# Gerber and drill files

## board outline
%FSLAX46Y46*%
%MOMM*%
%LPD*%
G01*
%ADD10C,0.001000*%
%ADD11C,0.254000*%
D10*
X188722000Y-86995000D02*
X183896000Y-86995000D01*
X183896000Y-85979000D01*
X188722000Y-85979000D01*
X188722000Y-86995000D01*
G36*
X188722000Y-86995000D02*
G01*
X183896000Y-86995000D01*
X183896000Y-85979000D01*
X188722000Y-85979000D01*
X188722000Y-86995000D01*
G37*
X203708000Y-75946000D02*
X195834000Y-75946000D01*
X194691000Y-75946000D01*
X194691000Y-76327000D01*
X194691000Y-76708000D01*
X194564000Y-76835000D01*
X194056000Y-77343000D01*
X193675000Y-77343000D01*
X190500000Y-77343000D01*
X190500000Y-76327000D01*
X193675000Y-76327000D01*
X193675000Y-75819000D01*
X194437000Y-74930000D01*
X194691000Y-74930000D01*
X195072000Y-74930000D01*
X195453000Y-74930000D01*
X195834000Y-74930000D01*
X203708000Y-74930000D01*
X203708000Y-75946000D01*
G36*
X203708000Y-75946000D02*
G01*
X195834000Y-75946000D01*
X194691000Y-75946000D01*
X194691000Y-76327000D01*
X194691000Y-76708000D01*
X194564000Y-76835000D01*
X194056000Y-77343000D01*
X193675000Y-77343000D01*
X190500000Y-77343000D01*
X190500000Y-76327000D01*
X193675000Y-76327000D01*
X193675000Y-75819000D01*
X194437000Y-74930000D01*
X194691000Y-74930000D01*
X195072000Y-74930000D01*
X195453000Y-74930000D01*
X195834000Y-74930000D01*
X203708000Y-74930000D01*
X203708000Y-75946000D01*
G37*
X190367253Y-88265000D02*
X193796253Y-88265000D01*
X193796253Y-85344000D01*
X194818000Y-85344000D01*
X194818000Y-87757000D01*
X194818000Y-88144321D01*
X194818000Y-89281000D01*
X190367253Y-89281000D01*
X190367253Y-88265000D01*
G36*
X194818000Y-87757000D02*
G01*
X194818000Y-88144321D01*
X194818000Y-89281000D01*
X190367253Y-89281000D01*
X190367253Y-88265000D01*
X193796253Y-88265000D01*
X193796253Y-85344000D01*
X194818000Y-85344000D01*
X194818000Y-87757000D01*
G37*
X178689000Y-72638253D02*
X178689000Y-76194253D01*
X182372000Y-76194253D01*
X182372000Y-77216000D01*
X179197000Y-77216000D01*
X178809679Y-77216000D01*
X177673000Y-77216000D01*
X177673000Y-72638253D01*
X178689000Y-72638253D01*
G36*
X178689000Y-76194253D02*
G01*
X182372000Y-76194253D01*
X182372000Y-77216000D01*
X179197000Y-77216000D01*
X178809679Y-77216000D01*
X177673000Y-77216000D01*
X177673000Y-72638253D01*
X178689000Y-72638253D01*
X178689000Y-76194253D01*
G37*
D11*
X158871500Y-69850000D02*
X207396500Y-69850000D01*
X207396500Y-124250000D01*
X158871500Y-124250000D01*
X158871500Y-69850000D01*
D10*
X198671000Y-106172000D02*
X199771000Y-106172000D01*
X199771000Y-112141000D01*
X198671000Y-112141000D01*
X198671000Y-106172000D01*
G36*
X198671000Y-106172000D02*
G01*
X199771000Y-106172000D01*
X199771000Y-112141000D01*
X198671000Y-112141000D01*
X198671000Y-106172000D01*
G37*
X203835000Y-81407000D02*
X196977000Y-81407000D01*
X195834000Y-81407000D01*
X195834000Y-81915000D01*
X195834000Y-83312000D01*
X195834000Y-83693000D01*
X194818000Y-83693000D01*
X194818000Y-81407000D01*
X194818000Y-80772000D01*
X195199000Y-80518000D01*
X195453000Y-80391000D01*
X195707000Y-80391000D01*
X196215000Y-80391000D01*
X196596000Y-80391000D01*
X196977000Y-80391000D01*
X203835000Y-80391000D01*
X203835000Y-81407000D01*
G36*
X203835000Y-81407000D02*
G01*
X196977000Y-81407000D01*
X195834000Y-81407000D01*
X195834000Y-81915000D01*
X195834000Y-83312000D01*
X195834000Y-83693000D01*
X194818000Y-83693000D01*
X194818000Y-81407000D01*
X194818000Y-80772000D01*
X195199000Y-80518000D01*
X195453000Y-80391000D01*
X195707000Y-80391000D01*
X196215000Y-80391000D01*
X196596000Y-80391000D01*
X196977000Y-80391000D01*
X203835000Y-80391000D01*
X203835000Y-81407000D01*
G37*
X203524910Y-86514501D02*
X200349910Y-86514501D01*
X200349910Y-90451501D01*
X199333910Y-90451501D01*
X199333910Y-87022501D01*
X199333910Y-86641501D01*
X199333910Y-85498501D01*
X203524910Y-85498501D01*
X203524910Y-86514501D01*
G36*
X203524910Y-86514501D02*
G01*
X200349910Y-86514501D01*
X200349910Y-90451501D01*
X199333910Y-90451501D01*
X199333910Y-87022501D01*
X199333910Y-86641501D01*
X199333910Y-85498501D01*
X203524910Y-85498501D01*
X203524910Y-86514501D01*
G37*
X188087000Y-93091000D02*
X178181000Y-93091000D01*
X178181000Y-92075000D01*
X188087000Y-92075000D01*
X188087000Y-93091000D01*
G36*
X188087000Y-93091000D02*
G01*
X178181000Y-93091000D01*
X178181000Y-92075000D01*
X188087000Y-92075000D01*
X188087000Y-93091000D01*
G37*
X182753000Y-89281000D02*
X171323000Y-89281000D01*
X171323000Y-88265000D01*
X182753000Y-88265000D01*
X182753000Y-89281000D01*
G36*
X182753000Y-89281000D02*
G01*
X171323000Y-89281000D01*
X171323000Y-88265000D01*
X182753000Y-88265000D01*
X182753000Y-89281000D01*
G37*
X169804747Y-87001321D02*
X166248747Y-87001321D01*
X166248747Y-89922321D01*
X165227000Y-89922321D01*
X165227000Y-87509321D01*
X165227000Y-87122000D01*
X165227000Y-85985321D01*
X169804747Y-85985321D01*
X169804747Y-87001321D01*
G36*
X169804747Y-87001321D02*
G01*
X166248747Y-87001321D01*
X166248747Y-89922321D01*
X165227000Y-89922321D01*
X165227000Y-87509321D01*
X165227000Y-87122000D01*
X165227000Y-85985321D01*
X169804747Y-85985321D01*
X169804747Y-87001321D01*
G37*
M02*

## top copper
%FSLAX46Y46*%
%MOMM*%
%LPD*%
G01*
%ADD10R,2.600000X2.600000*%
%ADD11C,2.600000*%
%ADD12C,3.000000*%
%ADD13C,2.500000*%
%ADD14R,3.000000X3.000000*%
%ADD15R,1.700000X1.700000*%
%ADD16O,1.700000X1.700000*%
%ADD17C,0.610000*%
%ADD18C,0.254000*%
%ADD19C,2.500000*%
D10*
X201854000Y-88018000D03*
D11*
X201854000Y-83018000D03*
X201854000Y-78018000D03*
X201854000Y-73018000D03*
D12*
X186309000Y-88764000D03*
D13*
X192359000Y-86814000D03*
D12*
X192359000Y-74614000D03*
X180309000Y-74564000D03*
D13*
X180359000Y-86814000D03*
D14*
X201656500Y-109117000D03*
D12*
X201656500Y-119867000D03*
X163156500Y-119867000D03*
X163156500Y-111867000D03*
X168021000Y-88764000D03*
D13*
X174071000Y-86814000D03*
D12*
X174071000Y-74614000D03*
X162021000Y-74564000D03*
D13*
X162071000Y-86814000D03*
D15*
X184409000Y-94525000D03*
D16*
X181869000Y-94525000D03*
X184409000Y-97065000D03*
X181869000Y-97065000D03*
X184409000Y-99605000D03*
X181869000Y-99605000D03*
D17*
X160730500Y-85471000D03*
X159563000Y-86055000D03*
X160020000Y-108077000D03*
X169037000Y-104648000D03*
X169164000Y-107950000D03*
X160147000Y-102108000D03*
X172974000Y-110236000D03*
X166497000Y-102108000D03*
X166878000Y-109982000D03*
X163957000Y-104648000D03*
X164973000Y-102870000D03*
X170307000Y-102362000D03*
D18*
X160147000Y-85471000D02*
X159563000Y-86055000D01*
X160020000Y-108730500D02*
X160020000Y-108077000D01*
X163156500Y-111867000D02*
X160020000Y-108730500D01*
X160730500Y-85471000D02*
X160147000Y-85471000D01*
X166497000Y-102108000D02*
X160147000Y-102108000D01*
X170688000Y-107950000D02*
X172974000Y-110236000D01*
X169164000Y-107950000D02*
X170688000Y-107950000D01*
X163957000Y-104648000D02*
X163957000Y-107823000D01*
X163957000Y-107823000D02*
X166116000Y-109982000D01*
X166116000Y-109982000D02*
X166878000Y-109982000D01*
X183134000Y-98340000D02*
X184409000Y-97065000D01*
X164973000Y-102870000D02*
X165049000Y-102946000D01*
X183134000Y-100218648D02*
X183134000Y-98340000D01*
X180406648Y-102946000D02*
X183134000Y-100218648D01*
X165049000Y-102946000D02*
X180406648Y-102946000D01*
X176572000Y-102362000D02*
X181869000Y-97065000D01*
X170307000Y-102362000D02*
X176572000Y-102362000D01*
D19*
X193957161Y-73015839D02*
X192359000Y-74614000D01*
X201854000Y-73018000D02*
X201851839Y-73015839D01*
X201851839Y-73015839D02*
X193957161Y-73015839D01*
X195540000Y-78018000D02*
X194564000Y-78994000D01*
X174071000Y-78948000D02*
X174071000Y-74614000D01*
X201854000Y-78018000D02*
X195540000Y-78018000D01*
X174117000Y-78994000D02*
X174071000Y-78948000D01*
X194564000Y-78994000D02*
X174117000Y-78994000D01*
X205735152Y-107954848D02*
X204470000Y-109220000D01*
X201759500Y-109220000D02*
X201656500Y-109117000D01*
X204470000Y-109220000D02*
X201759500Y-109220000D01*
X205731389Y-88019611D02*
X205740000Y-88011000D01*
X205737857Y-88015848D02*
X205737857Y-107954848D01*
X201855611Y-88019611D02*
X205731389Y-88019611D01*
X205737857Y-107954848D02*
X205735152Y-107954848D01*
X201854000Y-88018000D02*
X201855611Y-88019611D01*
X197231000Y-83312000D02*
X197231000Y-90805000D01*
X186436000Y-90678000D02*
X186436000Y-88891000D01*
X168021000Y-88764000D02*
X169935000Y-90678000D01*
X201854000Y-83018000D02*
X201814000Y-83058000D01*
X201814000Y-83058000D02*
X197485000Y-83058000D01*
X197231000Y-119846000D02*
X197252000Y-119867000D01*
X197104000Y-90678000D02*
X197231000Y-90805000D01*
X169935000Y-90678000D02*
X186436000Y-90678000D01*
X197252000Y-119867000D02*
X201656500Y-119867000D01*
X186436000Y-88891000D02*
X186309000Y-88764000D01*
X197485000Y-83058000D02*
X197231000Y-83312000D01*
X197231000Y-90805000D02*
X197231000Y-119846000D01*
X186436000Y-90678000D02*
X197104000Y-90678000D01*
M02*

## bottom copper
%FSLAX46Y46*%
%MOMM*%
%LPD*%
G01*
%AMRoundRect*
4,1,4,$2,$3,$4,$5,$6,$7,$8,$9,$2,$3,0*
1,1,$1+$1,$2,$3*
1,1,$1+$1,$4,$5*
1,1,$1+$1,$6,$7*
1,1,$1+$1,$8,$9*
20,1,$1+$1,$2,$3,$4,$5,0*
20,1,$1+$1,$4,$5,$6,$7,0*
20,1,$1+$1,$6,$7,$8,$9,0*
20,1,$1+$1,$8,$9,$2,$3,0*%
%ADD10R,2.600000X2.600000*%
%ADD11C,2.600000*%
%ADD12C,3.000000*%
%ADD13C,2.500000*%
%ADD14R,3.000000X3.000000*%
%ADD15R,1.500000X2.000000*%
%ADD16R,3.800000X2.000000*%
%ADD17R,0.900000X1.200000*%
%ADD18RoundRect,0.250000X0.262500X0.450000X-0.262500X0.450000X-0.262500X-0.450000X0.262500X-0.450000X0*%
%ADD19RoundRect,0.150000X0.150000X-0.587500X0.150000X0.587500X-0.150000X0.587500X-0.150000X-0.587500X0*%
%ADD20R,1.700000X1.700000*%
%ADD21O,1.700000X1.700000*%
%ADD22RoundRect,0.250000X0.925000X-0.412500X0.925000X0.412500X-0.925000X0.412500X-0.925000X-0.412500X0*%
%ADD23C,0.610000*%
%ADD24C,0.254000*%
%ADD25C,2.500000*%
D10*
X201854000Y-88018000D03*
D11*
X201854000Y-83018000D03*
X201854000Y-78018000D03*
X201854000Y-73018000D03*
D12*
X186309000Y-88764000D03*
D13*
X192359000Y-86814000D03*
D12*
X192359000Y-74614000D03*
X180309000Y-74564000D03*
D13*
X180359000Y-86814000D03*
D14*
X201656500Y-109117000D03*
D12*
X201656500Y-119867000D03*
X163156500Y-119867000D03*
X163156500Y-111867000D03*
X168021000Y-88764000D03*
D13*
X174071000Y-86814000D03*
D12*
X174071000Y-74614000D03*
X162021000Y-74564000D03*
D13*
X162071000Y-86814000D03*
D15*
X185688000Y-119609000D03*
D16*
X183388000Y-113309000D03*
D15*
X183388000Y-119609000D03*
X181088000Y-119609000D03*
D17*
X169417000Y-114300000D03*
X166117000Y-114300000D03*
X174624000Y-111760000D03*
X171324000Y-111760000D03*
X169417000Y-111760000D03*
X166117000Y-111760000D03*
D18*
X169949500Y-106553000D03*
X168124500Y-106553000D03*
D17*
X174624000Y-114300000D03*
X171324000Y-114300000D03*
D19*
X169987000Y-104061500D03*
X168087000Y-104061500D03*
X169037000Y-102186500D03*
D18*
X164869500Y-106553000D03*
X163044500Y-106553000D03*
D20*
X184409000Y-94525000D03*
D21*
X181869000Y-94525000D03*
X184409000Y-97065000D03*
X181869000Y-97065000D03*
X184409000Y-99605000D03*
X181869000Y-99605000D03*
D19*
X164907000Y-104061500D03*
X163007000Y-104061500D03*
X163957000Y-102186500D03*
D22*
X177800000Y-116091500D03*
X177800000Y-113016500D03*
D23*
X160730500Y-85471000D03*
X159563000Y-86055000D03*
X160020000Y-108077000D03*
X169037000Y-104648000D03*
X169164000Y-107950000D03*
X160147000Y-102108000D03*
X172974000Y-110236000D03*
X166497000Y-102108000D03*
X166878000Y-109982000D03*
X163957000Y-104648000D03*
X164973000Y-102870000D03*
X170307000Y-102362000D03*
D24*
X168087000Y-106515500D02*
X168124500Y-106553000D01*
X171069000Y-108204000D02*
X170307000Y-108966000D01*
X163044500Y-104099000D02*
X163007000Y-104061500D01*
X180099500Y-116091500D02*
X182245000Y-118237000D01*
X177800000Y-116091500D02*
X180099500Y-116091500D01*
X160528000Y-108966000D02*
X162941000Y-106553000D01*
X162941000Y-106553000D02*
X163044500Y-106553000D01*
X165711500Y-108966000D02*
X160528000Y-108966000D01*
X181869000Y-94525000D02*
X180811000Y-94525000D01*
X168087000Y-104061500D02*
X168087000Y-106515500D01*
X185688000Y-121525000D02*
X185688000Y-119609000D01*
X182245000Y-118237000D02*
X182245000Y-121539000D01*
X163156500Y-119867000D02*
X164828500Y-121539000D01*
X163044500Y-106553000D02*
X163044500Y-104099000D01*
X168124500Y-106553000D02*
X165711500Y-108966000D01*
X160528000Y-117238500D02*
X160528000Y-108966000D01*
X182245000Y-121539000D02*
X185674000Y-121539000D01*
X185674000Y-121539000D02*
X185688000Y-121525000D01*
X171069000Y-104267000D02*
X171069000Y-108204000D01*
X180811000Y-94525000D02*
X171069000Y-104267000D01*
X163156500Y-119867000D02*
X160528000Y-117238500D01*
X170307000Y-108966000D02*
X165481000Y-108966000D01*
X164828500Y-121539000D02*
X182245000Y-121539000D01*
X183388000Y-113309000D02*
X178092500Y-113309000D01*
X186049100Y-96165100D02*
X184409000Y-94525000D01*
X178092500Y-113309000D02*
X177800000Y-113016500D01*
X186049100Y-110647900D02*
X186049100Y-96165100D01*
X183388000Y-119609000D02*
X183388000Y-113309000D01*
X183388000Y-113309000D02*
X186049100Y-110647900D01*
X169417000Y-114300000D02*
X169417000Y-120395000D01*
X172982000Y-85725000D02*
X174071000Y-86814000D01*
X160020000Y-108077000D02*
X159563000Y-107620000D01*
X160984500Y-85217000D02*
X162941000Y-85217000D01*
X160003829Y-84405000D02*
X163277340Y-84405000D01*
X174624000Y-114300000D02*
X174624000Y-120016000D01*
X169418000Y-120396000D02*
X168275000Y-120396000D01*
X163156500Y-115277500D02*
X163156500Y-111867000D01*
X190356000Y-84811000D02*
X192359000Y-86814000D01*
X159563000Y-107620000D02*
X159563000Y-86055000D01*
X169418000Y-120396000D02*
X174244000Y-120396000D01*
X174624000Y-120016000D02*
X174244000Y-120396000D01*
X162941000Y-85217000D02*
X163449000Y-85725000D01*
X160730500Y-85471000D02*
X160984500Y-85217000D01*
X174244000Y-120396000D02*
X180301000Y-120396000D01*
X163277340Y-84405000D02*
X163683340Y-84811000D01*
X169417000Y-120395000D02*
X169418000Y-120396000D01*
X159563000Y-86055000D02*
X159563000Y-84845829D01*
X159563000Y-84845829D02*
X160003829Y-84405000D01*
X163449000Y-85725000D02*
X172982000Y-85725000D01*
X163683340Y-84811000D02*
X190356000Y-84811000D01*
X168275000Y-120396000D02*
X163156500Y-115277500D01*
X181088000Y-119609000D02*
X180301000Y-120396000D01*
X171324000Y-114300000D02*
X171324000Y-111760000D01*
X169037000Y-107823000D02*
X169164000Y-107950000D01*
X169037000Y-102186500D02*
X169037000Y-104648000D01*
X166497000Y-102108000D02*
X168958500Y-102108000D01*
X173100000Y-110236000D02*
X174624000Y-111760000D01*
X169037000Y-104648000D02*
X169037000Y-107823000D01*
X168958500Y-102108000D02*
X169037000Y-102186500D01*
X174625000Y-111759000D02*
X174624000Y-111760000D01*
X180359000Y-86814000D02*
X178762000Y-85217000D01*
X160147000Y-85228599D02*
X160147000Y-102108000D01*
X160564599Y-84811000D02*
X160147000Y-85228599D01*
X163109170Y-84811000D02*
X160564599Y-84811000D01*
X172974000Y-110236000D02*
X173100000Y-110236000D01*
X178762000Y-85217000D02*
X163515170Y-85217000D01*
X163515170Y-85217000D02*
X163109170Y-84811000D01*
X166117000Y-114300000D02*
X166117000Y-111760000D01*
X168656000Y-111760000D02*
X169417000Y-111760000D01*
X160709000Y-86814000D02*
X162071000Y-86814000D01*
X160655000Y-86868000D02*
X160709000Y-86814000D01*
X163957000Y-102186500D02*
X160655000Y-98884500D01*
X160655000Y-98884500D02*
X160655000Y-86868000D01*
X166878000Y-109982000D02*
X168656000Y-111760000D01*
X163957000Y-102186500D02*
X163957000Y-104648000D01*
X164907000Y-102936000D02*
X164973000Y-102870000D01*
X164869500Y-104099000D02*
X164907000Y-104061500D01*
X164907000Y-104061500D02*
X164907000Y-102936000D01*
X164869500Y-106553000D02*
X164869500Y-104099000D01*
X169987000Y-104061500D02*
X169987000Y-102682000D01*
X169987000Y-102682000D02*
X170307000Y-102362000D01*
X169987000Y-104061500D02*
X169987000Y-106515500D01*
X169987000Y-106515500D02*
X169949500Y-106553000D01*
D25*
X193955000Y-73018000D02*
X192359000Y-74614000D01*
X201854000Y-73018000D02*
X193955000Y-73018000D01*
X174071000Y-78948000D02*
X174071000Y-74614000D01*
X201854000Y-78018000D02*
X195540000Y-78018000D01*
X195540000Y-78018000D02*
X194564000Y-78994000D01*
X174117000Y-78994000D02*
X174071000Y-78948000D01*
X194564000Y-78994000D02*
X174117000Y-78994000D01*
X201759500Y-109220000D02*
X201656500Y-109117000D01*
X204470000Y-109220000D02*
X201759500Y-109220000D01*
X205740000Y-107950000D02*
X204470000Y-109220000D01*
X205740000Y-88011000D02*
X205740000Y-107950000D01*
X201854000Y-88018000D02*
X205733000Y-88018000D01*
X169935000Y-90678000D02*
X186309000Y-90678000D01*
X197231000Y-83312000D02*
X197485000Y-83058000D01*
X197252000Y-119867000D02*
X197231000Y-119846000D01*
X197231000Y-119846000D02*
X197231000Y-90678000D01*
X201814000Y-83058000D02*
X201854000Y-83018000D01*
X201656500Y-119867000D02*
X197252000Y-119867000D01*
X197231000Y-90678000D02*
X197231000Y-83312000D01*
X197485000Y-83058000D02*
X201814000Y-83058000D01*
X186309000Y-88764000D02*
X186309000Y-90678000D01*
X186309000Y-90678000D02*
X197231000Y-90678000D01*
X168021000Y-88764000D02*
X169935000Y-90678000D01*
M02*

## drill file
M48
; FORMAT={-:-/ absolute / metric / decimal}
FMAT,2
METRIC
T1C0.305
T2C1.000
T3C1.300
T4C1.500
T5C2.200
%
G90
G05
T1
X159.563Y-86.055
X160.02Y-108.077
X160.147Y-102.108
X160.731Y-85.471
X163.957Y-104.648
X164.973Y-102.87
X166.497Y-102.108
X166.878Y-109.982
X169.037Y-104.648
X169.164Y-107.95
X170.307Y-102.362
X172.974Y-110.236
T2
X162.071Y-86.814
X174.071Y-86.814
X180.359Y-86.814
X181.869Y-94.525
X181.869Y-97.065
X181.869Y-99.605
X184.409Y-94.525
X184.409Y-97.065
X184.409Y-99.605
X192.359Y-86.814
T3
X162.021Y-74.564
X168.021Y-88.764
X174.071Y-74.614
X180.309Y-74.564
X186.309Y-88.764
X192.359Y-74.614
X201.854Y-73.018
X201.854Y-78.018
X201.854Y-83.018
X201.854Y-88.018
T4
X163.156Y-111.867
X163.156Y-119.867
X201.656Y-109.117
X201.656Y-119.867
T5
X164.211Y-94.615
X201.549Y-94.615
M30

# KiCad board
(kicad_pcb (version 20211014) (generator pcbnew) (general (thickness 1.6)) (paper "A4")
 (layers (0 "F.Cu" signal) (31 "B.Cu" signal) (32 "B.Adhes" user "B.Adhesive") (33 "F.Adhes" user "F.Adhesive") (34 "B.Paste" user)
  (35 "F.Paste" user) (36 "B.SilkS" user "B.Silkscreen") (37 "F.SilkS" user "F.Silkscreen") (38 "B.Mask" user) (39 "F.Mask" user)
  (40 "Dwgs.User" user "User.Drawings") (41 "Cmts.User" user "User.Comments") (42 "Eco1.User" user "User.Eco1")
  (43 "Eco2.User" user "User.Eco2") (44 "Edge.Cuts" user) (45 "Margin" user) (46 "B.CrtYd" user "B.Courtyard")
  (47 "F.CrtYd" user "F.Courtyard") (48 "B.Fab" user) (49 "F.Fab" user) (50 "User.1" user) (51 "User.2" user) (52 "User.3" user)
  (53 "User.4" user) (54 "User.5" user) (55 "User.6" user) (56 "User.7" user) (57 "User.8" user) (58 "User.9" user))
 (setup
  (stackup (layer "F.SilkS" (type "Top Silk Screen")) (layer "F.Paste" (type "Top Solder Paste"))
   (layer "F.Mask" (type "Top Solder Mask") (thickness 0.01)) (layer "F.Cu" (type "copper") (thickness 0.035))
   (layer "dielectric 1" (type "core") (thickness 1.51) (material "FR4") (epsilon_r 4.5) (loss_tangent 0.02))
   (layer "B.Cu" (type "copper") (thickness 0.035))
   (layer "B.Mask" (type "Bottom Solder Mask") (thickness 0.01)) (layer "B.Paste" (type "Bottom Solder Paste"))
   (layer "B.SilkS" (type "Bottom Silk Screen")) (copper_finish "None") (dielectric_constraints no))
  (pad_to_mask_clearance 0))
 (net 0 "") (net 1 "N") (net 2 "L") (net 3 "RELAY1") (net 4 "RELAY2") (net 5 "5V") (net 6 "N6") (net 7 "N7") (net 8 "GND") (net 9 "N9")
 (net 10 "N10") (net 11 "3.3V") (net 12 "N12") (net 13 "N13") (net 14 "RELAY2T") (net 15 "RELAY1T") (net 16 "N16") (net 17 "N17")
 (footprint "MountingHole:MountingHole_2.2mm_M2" (layer "F.Cu") (at 164.211 94.615)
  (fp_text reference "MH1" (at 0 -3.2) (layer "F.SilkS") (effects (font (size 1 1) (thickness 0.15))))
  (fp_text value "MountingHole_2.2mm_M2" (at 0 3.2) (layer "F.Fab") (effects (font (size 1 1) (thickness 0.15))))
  (pad "" np_thru_hole circle (at 0 0) (size 2.2 2.2) (drill 2.2) (layers *.Cu *.Mask)))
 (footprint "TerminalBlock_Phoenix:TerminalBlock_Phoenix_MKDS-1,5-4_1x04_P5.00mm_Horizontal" (layer "F.Cu") (at 201.854 88.018 90)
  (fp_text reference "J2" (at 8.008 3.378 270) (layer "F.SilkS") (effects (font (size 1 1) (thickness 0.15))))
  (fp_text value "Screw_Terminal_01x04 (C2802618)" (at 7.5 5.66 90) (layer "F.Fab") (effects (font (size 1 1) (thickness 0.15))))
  (pad "1" thru_hole rect (at 0 0 90) (size 2.6 2.6) (drill 1.3) (layers *.Cu *.Mask) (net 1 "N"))
  (pad "2" thru_hole circle (at 5 0 90) (size 2.6 2.6) (drill 1.3) (layers *.Cu *.Mask) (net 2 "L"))
  (pad "3" thru_hole circle (at 10 0 90) (size 2.6 2.6) (drill 1.3) (layers *.Cu *.Mask) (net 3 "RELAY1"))
  (pad "4" thru_hole circle (at 15 0 90) (size 2.6 2.6) (drill 1.3) (layers *.Cu *.Mask) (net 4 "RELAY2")))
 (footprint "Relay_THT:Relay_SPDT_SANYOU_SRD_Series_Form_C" (layer "F.Cu") (at 186.309 88.764 90)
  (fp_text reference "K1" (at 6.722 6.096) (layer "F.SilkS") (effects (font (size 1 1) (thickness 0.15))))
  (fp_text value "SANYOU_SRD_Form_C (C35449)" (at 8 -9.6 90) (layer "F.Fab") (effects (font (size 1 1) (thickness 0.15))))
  (pad "1" thru_hole circle (at 0 0 180) (size 3 3) (drill 1.3) (layers *.Cu *.Mask) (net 2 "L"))
  (pad "2" thru_hole circle (at 1.95 6.05 180) (size 2.5 2.5) (drill 1) (layers *.Cu *.Mask) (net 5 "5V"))
  (pad "3" thru_hole circle (at 14.15 6.05 180) (size 3 3) (drill 1.3) (layers *.Cu *.Mask) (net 4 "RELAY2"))
  (pad "4" thru_hole circle (at 14.2 -6 180) (size 3 3) (drill 1.3) (layers *.Cu *.Mask) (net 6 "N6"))
  (pad "5" thru_hole circle (at 1.95 -5.95 180) (size 2.5 2.5) (drill 1) (layers *.Cu *.Mask) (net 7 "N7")))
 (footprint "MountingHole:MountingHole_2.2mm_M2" (layer "F.Cu") (at 201.549 94.615)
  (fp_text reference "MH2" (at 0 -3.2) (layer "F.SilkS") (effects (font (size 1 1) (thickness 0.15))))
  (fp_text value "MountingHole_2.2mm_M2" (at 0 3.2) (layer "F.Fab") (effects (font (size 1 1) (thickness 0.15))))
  (pad "" np_thru_hole circle (at 0 0) (size 2.2 2.2) (drill 2.2) (layers *.Cu *.Mask)))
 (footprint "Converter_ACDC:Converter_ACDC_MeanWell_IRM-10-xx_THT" (layer "F.Cu") (at 161.0165 109.117)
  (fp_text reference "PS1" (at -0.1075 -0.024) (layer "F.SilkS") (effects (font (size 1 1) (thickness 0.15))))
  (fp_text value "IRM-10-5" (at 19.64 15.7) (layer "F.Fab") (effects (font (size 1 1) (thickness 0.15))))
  (pad "1" thru_hole rect (at 40.64 0) (size 3 3) (drill 1.5) (layers *.Cu *.Mask) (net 1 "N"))
  (pad "2" thru_hole circle (at 40.64 10.75) (size 3 3) (drill 1.5) (layers *.Cu *.Mask) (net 2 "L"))
  (pad "3" thru_hole circle (at 2.14 10.75) (size 3 3) (drill 1.5) (layers *.Cu *.Mask) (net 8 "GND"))
  (pad "4" thru_hole circle (at 2.14 2.75) (size 3 3) (drill 1.5) (layers *.Cu *.Mask) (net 5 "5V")))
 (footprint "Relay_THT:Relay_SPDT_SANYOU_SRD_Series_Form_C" (layer "F.Cu") (at 168.021 88.764 90)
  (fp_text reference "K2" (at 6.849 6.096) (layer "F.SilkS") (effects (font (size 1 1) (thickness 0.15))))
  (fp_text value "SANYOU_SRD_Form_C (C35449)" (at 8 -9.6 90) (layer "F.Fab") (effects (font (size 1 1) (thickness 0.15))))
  (pad "1" thru_hole circle (at 0 0 180) (size 3 3) (drill 1.3) (layers *.Cu *.Mask) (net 2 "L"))
  (pad "2" thru_hole circle (at 1.95 6.05 180) (size 2.5 2.5) (drill 1) (layers *.Cu *.Mask) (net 5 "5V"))
  (pad "3" thru_hole circle (at 14.15 6.05 180) (size 3 3) (drill 1.3) (layers *.Cu *.Mask) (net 3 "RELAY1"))
  (pad "4" thru_hole circle (at 14.2 -6 180) (size 3 3) (drill 1.3) (layers *.Cu *.Mask) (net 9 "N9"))
  (pad "5" thru_hole circle (at 1.95 -5.95 180) (size 2.5 2.5) (drill 1) (layers *.Cu *.Mask) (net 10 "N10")))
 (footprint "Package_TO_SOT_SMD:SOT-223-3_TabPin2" (layer "B.Cu") (at 183.388 116.459 90)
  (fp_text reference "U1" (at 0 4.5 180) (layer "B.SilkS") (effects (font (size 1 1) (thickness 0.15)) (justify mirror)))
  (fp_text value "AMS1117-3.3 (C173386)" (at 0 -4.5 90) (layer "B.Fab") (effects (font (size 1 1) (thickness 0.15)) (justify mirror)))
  (pad "1" smd rect (at -3.15 2.3 90) (size 2 1.5) (layers "B.Cu" "B.Paste" "B.Mask") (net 8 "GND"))
  (pad "2" smd rect (at 3.15 0 90) (size 2 3.8) (layers "B.Cu" "B.Paste" "B.Mask") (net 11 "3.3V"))
  (pad "2" smd rect (at -3.15 0 90) (size 2 1.5) (layers "B.Cu" "B.Paste" "B.Mask") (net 11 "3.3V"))
  (pad "3" smd rect (at -3.15 -2.3 90) (size 2 1.5) (layers "B.Cu" "B.Paste" "B.Mask") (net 5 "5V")))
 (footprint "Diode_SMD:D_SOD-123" (layer "B.Cu") (at 167.767 114.3 180)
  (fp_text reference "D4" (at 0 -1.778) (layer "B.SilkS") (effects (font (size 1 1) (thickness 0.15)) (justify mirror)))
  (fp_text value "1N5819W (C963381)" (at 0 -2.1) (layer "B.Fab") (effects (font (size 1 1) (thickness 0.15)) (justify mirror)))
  (pad "1" smd rect (at -1.65 0 180) (size 0.9 1.2) (layers "B.Cu" "B.Paste" "B.Mask") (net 5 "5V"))
  (pad "2" smd rect (at 1.65 0 180) (size 0.9 1.2) (layers "B.Cu" "B.Paste" "B.Mask") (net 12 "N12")))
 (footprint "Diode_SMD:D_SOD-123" (layer "B.Cu") (at 172.974 111.76 180)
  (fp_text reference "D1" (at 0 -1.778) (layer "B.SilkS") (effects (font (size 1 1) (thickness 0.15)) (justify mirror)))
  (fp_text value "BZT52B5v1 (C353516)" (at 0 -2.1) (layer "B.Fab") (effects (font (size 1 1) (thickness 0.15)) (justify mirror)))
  (pad "1" smd rect (at -1.65 0 180) (size 0.9 1.2) (layers "B.Cu" "B.Paste" "B.Mask") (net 7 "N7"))
  (pad "2" smd rect (at 1.65 0 180) (size 0.9 1.2) (layers "B.Cu" "B.Paste" "B.Mask") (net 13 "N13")))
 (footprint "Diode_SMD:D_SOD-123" (layer "B.Cu") (at 167.767 111.76 180)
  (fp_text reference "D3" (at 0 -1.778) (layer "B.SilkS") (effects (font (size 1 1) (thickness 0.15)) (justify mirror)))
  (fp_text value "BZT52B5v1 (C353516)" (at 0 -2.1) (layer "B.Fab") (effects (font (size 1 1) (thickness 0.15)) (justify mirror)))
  (pad "1" smd rect (at -1.65 0 180) (size 0.9 1.2) (layers "B.Cu" "B.Paste" "B.Mask") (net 10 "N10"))
  (pad "2" smd rect (at 1.65 0 180) (size 0.9 1.2) (layers "B.Cu" "B.Paste" "B.Mask") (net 12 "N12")))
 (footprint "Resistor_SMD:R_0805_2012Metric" (layer "B.Cu") (at 169.037 106.553 180)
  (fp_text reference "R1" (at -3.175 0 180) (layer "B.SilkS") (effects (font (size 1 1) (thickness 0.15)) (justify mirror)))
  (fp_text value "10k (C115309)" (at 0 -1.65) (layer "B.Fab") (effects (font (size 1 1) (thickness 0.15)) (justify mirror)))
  (pad "1" smd roundrect (at -0.9125 0 180) (size 1.025 1.4) (layers "B.Cu" "B.Paste" "B.Mask") (roundrect_rratio 0.243902)
   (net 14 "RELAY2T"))
  (pad "2" smd roundrect (at 0.9125 0 180) (size 1.025 1.4) (layers "B.Cu" "B.Paste" "B.Mask") (roundrect_rratio 0.243902) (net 8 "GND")))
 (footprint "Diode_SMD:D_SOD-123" (layer "B.Cu") (at 172.974 114.3 180)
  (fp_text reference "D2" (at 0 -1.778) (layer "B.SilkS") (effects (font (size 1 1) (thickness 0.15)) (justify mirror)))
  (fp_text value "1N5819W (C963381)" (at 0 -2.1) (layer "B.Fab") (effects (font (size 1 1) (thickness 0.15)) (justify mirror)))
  (pad "1" smd rect (at -1.65 0 180) (size 0.9 1.2) (layers "B.Cu" "B.Paste" "B.Mask") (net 5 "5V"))
  (pad "2" smd rect (at 1.65 0 180) (size 0.9 1.2) (layers "B.Cu" "B.Paste" "B.Mask") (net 13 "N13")))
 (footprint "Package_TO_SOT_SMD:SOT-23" (layer "B.Cu") (at 169.037 103.124 90)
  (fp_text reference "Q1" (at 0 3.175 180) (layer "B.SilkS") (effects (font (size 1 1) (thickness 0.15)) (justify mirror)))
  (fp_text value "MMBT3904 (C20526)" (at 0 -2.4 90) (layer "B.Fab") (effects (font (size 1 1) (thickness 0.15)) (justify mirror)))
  (pad "1" smd roundrect (at -0.9375 0.95 90) (size 1.475 0.6) (layers "B.Cu" "B.Paste" "B.Mask") (roundrect_rratio 0.25) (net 14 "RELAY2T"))
  (pad "2" smd roundrect (at -0.9375 -0.95 90) (size 1.475 0.6) (layers "B.Cu" "B.Paste" "B.Mask") (roundrect_rratio 0.25) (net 8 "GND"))
  (pad "3" smd roundrect (at 0.9375 0 90) (size 1.475 0.6) (layers "B.Cu" "B.Paste" "B.Mask") (roundrect_rratio 0.25) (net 7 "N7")))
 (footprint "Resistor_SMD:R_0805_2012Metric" (layer "B.Cu") (at 163.957 106.553 180)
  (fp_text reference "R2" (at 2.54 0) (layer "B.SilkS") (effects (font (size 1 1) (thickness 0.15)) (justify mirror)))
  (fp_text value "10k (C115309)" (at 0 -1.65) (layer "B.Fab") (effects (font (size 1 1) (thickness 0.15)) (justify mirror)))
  (pad "1" smd roundrect (at -0.9125 0 180) (size 1.025 1.4) (layers "B.Cu" "B.Paste" "B.Mask") (roundrect_rratio 0.243902)
   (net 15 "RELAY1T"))
  (pad "2" smd roundrect (at 0.9125 0 180) (size 1.025 1.4) (layers "B.Cu" "B.Paste" "B.Mask") (roundrect_rratio 0.243902) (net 8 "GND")))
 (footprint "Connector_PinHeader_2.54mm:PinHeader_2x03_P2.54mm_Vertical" (layer "B.Cu") (at 184.409 94.525 180)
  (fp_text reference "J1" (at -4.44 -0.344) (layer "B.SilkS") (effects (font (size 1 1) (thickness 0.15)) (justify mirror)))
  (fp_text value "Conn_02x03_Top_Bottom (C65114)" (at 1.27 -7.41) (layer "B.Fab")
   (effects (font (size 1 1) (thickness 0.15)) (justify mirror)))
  (pad "1" thru_hole rect (at 0 0 180) (size 1.7 1.7) (drill 1) (layers *.Cu *.Mask) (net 11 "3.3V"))
  (pad "2" thru_hole oval (at 2.54 0 180) (size 1.7 1.7) (drill 1) (layers *.Cu *.Mask) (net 8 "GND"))
  (pad "3" thru_hole oval (at 0 -2.54 180) (size 1.7 1.7) (drill 1) (layers *.Cu *.Mask) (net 15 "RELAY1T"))
  (pad "4" thru_hole oval (at 2.54 -2.54 180) (size 1.7 1.7) (drill 1) (layers *.Cu *.Mask) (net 14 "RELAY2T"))
  (pad "5" thru_hole oval (at 0 -5.08 180) (size 1.7 1.7) (drill 1) (layers *.Cu *.Mask) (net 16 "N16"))
  (pad "6" thru_hole oval (at 2.54 -5.08 180) (size 1.7 1.7) (drill 1) (layers *.Cu *.Mask) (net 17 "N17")))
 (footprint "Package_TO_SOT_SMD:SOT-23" (layer "B.Cu") (at 163.957 103.124 90)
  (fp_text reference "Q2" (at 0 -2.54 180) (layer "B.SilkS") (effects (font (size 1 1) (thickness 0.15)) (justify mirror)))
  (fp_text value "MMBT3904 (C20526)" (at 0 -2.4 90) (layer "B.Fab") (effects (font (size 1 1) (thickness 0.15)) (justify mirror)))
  (pad "1" smd roundrect (at -0.9375 0.95 90) (size 1.475 0.6) (layers "B.Cu" "B.Paste" "B.Mask") (roundrect_rratio 0.25) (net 15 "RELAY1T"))
  (pad "2" smd roundrect (at -0.9375 -0.95 90) (size 1.475 0.6) (layers "B.Cu" "B.Paste" "B.Mask") (roundrect_rratio 0.25) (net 8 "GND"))
  (pad "3" smd roundrect (at 0.9375 0 90) (size 1.475 0.6) (layers "B.Cu" "B.Paste" "B.Mask") (roundrect_rratio 0.25) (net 10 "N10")))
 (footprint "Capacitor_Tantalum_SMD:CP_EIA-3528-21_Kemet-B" (layer "B.Cu") (at 177.8 114.554 90)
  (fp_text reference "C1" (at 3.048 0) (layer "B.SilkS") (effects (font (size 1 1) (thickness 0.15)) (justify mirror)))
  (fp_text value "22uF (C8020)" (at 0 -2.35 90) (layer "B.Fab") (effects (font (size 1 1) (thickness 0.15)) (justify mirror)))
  (pad "1" smd roundrect (at -1.5375 0 90) (size 1.325 2.35) (layers "B.Cu" "B.Paste" "B.Mask") (roundrect_rratio 0.188679) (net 8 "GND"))
  (pad "2" smd roundrect (at 1.5375 0 90) (size 1.325 2.35) (layers "B.Cu" "B.Paste" "B.Mask") (roundrect_rratio 0.188679) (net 11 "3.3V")))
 (gr_poly
  (pts (xy 188.722 86.995) (xy 183.896 86.995) (xy 183.896 85.979) (xy 188.722 85.979)) (layer "Edge.Cuts") (width 0.001) (fill solid))
 (gr_poly
  (pts (xy 203.708 75.946) (xy 195.834 75.946) (xy 194.691 75.946) (xy 194.691 76.327) (xy 194.691 76.708) (xy 194.564 76.835)
   (xy 194.056 77.343) (xy 193.675 77.343) (xy 190.5 77.343) (xy 190.5 76.327) (xy 193.675 76.327) (xy 193.675 75.819) (xy 194.437 74.93)
   (xy 194.691 74.93) (xy 195.072 74.93) (xy 195.453 74.93) (xy 195.834 74.93) (xy 203.708 74.93))
  (layer "Edge.Cuts") (width 0.001) (fill solid))
 (gr_poly
  (pts (xy 190.367253 88.265) (xy 193.796253 88.265) (xy 193.796253 85.344) (xy 194.818 85.344) (xy 194.818 87.757) (xy 194.818 88.144321)
   (xy 194.818 89.281) (xy 190.367253 89.281))
  (layer "Edge.Cuts") (width 0.001) (fill solid))
 (gr_poly
  (pts (xy 178.689 72.638253) (xy 178.689 76.194253) (xy 182.372 76.194253) (xy 182.372 77.216) (xy 179.197 77.216) (xy 178.809679 77.216)
   (xy 177.673 77.216) (xy 177.673 72.638253))
  (layer "Edge.Cuts") (width 0.001) (fill solid))
 (gr_rect (start 158.8715 69.85) (end 207.3965 124.25) (layer "Edge.Cuts") (width 0.254) (fill none))
 (gr_rect (start 198.671 112.141) (end 199.771 106.172) (layer "Edge.Cuts") (width 0.001) (fill solid))
 (gr_poly
  (pts (xy 203.835 81.407) (xy 196.977 81.407) (xy 195.834 81.407) (xy 195.834 81.915) (xy 195.834 83.312) (xy 195.834 83.693)
   (xy 194.818 83.693) (xy 194.818 81.407) (xy 194.818 80.772) (xy 195.199 80.518) (xy 195.453 80.391) (xy 195.707 80.391)
   (xy 196.215 80.391) (xy 196.596 80.391) (xy 196.977 80.391) (xy 203.835 80.391))
  (layer "Edge.Cuts") (width 0.001) (fill solid))
 (gr_poly
  (pts (xy 203.52491 86.514501) (xy 200.34991 86.514501) (xy 200.34991 90.451501) (xy 199.33391 90.451501) (xy 199.33391 87.022501)
   (xy 199.33391 86.641501) (xy 199.33391 85.498501) (xy 203.52491 85.498501))
  (layer "Edge.Cuts") (width 0.001) (fill solid))
 (gr_poly
  (pts (xy 188.087 93.091) (xy 178.181 93.091) (xy 178.181 92.075) (xy 188.087 92.075)) (layer "Edge.Cuts") (width 0.001) (fill solid))
 (gr_poly
  (pts (xy 182.753 89.281) (xy 171.323 89.281) (xy 171.323 88.265) (xy 182.753 88.265)) (layer "Edge.Cuts") (width 0.001) (fill solid))
 (gr_poly
  (pts (xy 169.804747 87.001321) (xy 166.248747 87.001321) (xy 166.248747 89.922321) (xy 165.227 89.922321) (xy 165.227 87.509321)
   (xy 165.227 87.122) (xy 165.227 85.985321) (xy 169.804747 85.985321))
  (layer "Edge.Cuts") (width 0.001) (fill solid))
 (segment (start 168.087 106.5155) (end 168.1245 106.553) (width 0.254) (layer "B.Cu") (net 8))
 (segment (start 171.069 108.204) (end 170.307 108.966) (width 0.254) (layer "B.Cu") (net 8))
 (segment (start 163.0445 104.099) (end 163.007 104.0615) (width 0.254) (layer "B.Cu") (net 8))
 (segment (start 180.0995 116.0915) (end 182.245 118.237) (width 0.254) (layer "B.Cu") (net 8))
 (segment (start 177.8 116.0915) (end 180.0995 116.0915) (width 0.254) (layer "B.Cu") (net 8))
 (segment (start 160.528 108.966) (end 162.941 106.553) (width 0.254) (layer "B.Cu") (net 8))
 (segment (start 162.941 106.553) (end 163.0445 106.553) (width 0.254) (layer "B.Cu") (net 8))
 (segment (start 165.7115 108.966) (end 160.528 108.966) (width 0.254) (layer "B.Cu") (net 8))
 (segment (start 181.869 94.525) (end 180.811 94.525) (width 0.254) (layer "B.Cu") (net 8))
 (segment (start 168.087 104.0615) (end 168.087 106.5155) (width 0.254) (layer "B.Cu") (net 8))
 (segment (start 185.688 121.525) (end 185.688 119.609) (width 0.254) (layer "B.Cu") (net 8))
 (segment (start 182.245 118.237) (end 182.245 121.539) (width 0.254) (layer "B.Cu") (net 8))
 (segment (start 163.1565 119.867) (end 164.8285 121.539) (width 0.254) (layer "B.Cu") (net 8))
 (segment (start 163.0445 106.553) (end 163.0445 104.099) (width 0.254) (layer "B.Cu") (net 8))
 (segment (start 168.1245 106.553) (end 165.7115 108.966) (width 0.254) (layer "B.Cu") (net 8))
 (segment (start 160.528 117.2385) (end 160.528 108.966) (width 0.254) (layer "B.Cu") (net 8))
 (segment (start 182.245 121.539) (end 185.674 121.539) (width 0.254) (layer "B.Cu") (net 8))
 (segment (start 185.674 121.539) (end 185.688 121.525) (width 0.254) (layer "B.Cu") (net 8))
 (segment (start 171.069 104.267) (end 171.069 108.204) (width 0.254) (layer "B.Cu") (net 8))
 (segment (start 180.811 94.525) (end 171.069 104.267) (width 0.254) (layer "B.Cu") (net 8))
 (segment (start 163.1565 119.867) (end 160.528 117.2385) (width 0.254) (layer "B.Cu") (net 8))
 (segment (start 170.307 108.966) (end 165.481 108.966) (width 0.254) (layer "B.Cu") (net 8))
 (segment (start 164.8285 121.539) (end 182.245 121.539) (width 0.254) (layer "B.Cu") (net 8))
 (segment (start 183.388 113.309) (end 178.0925 113.309) (width 0.254) (layer "B.Cu") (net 11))
 (segment (start 186.0491 96.1651) (end 184.409 94.525) (width 0.254) (layer "B.Cu") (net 11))
 (segment (start 178.0925 113.309) (end 177.8 113.0165) (width 0.254) (layer "B.Cu") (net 11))
 (segment (start 186.0491 110.6479) (end 186.0491 96.1651) (width 0.254) (layer "B.Cu") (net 11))
 (segment (start 183.388 119.609) (end 183.388 113.309) (width 0.254) (layer "B.Cu") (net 11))
 (segment (start 183.388 113.309) (end 186.0491 110.6479) (width 0.254) (layer "B.Cu") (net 11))
 (segment (start 160.147 85.471) (end 159.563 86.055) (width 0.254) (layer "F.Cu") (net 5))
 (segment (start 160.02 108.7305) (end 160.02 108.077) (width 0.254) (layer "F.Cu") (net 5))
 (segment (start 163.1565 111.867) (end 160.02 108.7305) (width 0.254) (layer "F.Cu") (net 5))
 (segment (start 160.7305 85.471) (end 160.147 85.471) (width 0.254) (layer "F.Cu") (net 5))
 (via (at 160.7305 85.471) (size 0.61) (drill 0.305) (layers "F.Cu" "B.Cu") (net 5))
 (via (at 159.563 86.055) (size 0.61) (drill 0.305) (layers "F.Cu" "B.Cu") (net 5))
 (via (at 160.02 108.077) (size 0.61) (drill 0.305) (layers "F.Cu" "B.Cu") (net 5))
 (segment (start 169.417 114.3) (end 169.417 120.395) (width 0.254) (layer "B.Cu") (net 5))
 (segment (start 172.982 85.725) (end 174.071 86.814) (width 0.254) (layer "B.Cu") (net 5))
 (segment (start 160.02 108.077) (end 159.563 107.62) (width 0.254) (layer "B.Cu") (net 5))
 (segment (start 160.9845 85.217) (end 162.941 85.217) (width 0.254) (layer "B.Cu") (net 5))
 (segment (start 160.003829 84.405) (end 163.27734 84.405) (width 0.254) (layer "B.Cu") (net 5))
 (segment (start 174.624 114.3) (end 174.624 120.016) (width 0.254) (layer "B.Cu") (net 5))
 (segment (start 169.418 120.396) (end 168.275 120.396) (width 0.254) (layer "B.Cu") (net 5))
 (segment (start 163.1565 115.2775) (end 163.1565 111.867) (width 0.254) (layer "B.Cu") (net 5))
 (segment (start 190.356 84.811) (end 192.359 86.814) (width 0.254) (layer "B.Cu") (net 5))
 (segment (start 159.563 107.62) (end 159.563 86.055) (width 0.254) (layer "B.Cu") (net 5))
 (segment (start 169.418 120.396) (end 174.244 120.396) (width 0.254) (layer "B.Cu") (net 5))
 (segment (start 174.624 120.016) (end 174.244 120.396) (width 0.254) (layer "B.Cu") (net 5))
 (segment (start 162.941 85.217) (end 163.449 85.725) (width 0.254) (layer "B.Cu") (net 5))
 (segment (start 160.7305 85.471) (end 160.9845 85.217) (width 0.254) (layer "B.Cu") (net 5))
 (segment (start 174.244 120.396) (end 180.301 120.396) (width 0.254) (layer "B.Cu") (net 5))
 (segment (start 163.27734 84.405) (end 163.68334 84.811) (width 0.254) (layer "B.Cu") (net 5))
 (segment (start 169.417 120.395) (end 169.418 120.396) (width 0.254) (layer "B.Cu") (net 5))
 (segment (start 159.563 86.055) (end 159.563 84.845829) (width 0.254) (layer "B.Cu") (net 5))
 (segment (start 159.563 84.845829) (end 160.003829 84.405) (width 0.254) (layer "B.Cu") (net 5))
 (segment (start 163.449 85.725) (end 172.982 85.725) (width 0.254) (layer "B.Cu") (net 5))
 (segment (start 163.68334 84.811) (end 190.356 84.811) (width 0.254) (layer "B.Cu") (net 5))
 (segment (start 168.275 120.396) (end 163.1565 115.2775) (width 0.254) (layer "B.Cu") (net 5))
 (segment (start 181.088 119.609) (end 180.301 120.396) (width 0.254) (layer "B.Cu") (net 5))
 (segment (start 171.324 114.3) (end 171.324 111.76) (width 0.254) (layer "B.Cu") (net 13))
 (segment (start 166.497 102.108) (end 160.147 102.108) (width 0.254) (layer "F.Cu") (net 7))
 (segment (start 170.688 107.95) (end 172.974 110.236) (width 0.254) (layer "F.Cu") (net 7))
 (segment (start 169.164 107.95) (end 170.688 107.95) (width 0.254) (layer "F.Cu") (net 7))
 (via (at 169.037 104.648) (size 0.61) (drill 0.305) (layers "F.Cu" "B.Cu") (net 7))
 (via (at 169.164 107.95) (size 0.61) (drill 0.305) (layers "F.Cu" "B.Cu") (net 7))
 (via (at 160.147 102.108) (size 0.61) (drill 0.305) (layers "F.Cu" "B.Cu") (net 7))
 (via (at 172.974 110.236) (size 0.61) (drill 0.305) (layers "F.Cu" "B.Cu") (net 7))
 (via (at 166.497 102.108) (size 0.61) (drill 0.305) (layers "F.Cu" "B.Cu") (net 7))
 (segment (start 169.037 107.823) (end 169.164 107.95) (width 0.254) (layer "B.Cu") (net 7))
 (segment (start 169.037 102.1865) (end 169.037 104.648) (width 0.254) (layer "B.Cu") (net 7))
 (segment (start 166.497 102.108) (end 168.9585 102.108) (width 0.254) (layer "B.Cu") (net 7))
 (segment (start 173.1 110.236) (end 174.624 111.76) (width 0.254) (layer "B.Cu") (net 7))
 (segment (start 169.037 104.648) (end 169.037 107.823) (width 0.254) (layer "B.Cu") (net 7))
 (segment (start 168.9585 102.108) (end 169.037 102.1865) (width 0.254) (layer "B.Cu") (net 7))
 (segment (start 174.625 111.759) (end 174.624 111.76) (width 0.254) (layer "B.Cu") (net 7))
 (segment (start 180.359 86.814) (end 178.762 85.217) (width 0.254) (layer "B.Cu") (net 7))
 (segment (start 160.147 85.228599) (end 160.147 102.108) (width 0.254) (layer "B.Cu") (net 7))
 (segment (start 160.564599 84.811) (end 160.147 85.228599) (width 0.254) (layer "B.Cu") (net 7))
 (segment (start 163.10917 84.811) (end 160.564599 84.811) (width 0.254) (layer "B.Cu") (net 7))
 (segment (start 172.974 110.236) (end 173.1 110.236) (width 0.254) (layer "B.Cu") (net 7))
 (segment (start 178.762 85.217) (end 163.51517 85.217) (width 0.254) (layer "B.Cu") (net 7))
 (segment (start 163.51517 85.217) (end 163.10917 84.811) (width 0.254) (layer "B.Cu") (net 7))
 (segment (start 166.117 114.3) (end 166.117 111.76) (width 0.254) (layer "B.Cu") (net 12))
 (segment (start 163.957 104.648) (end 163.957 107.823) (width 0.254) (layer "F.Cu") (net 10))
 (segment (start 163.957 107.823) (end 166.116 109.982) (width 0.254) (layer "F.Cu") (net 10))
 (segment (start 166.116 109.982) (end 166.878 109.982) (width 0.254) (layer "F.Cu") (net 10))
 (via (at 166.878 109.982) (size 0.61) (drill 0.305) (layers "F.Cu" "B.Cu") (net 10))
 (via (at 163.957 104.648) (size 0.61) (drill 0.305) (layers "F.Cu" "B.Cu") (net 10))
 (segment (start 168.656 111.76) (end 169.417 111.76) (width 0.254) (layer "B.Cu") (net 10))
 (segment (start 160.709 86.814) (end 162.071 86.814) (width 0.254) (layer "B.Cu") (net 10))
 (segment (start 160.655 86.868) (end 160.709 86.814) (width 0.254) (layer "B.Cu") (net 10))
 (segment (start 163.957 102.1865) (end 160.655 98.8845) (width 0.254) (layer "B.Cu") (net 10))
 (segment (start 160.655 98.8845) (end 160.655 86.868) (width 0.254) (layer "B.Cu") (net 10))
 (segment (start 166.878 109.982) (end 168.656 111.76) (width 0.254) (layer "B.Cu") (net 10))
 (segment (start 163.957 102.1865) (end 163.957 104.648) (width 0.254) (layer "B.Cu") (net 10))
 (segment (start 183.134 98.34) (end 184.409 97.065) (width 0.254) (layer "F.Cu") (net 15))
 (segment (start 164.973 102.87) (end 165.049 102.946) (width 0.254) (layer "F.Cu") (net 15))
 (segment (start 183.134 100.218648) (end 183.134 98.34) (width 0.254) (layer "F.Cu") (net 15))
 (segment (start 180.406648 102.946) (end 183.134 100.218648) (width 0.254) (layer "F.Cu") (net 15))
 (segment (start 165.049 102.946) (end 180.406648 102.946) (width 0.254) (layer "F.Cu") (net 15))
 (via (at 164.973 102.87) (size 0.61) (drill 0.305) (layers "F.Cu" "B.Cu") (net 15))
 (segment (start 164.907 102.936) (end 164.973 102.87) (width 0.254) (layer "B.Cu") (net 15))
 (segment (start 164.8695 104.099) (end 164.907 104.0615) (width 0.254) (layer "B.Cu") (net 15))
 (segment (start 164.907 104.0615) (end 164.907 102.936) (width 0.254) (layer "B.Cu") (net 15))
 (segment (start 164.8695 106.553) (end 164.8695 104.099) (width 0.254) (layer "B.Cu") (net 15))
 (segment (start 176.572 102.362) (end 181.869 97.065) (width 0.254) (layer "F.Cu") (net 14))
 (segment (start 170.307 102.362) (end 176.572 102.362) (width 0.254) (layer "F.Cu") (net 14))
 (via (at 170.307 102.362) (size 0.61) (drill 0.305) (layers "F.Cu" "B.Cu") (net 14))
 (segment (start 169.987 104.0615) (end 169.987 102.682) (width 0.254) (layer "B.Cu") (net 14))
 (segment (start 169.987 102.682) (end 170.307 102.362) (width 0.254) (layer "B.Cu") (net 14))
 (segment (start 169.987 104.0615) (end 169.987 106.5155) (width 0.254) (layer "B.Cu") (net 14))
 (segment (start 169.987 106.5155) (end 169.9495 106.553) (width 0.254) (layer "B.Cu") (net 14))
 (segment (start 193.957161 73.015839) (end 192.359 74.614) (width 2.5) (layer "F.Cu") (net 4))
 (segment (start 201.854 73.018) (end 201.851839 73.015839) (width 2.5) (layer "F.Cu") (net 4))
 (segment (start 201.851839 73.015839) (end 193.957161 73.015839) (width 2.5) (layer "F.Cu") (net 4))
 (segment (start 193.955 73.018) (end 192.359 74.614) (width 2.5) (layer "B.Cu") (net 4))
 (segment (start 201.854 73.018) (end 193.955 73.018) (width 2.5) (layer "B.Cu") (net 4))
 (segment (start 195.54 78.018) (end 194.564 78.994) (width 2.5) (layer "F.Cu") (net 3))
 (segment (start 174.071 78.948) (end 174.071 74.614) (width 2.5) (layer "F.Cu") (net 3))
 (segment (start 201.854 78.018) (end 195.54 78.018) (width 2.5) (layer "F.Cu") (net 3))
 (segment (start 174.117 78.994) (end 174.071 78.948) (width 2.5) (layer "F.Cu") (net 3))
 (segment (start 194.564 78.994) (end 174.117 78.994) (width 2.5) (layer "F.Cu") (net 3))
 (segment (start 174.071 78.948) (end 174.071 74.614) (width 2.5) (layer "B.Cu") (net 3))
 (segment (start 201.854 78.018) (end 195.54 78.018) (width 2.5) (layer "B.Cu") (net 3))
 (segment (start 195.54 78.018) (end 194.564 78.994) (width 2.5) (layer "B.Cu") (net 3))
 (segment (start 174.117 78.994) (end 174.071 78.948) (width 2.5) (layer "B.Cu") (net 3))
 (segment (start 194.564 78.994) (end 174.117 78.994) (width 2.5) (layer "B.Cu") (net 3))
 (segment (start 205.735152 107.954848) (end 204.47 109.22) (width 2.5) (layer "F.Cu") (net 1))
 (segment (start 201.7595 109.22) (end 201.6565 109.117) (width 2.5) (layer "F.Cu") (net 1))
 (segment (start 204.47 109.22) (end 201.7595 109.22) (width 2.5) (layer "F.Cu") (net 1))
 (segment (start 205.731389 88.019611) (end 205.74 88.011) (width 2.5) (layer "F.Cu") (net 1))
 (segment (start 205.737857 88.015848) (end 205.737857 107.954848) (width 2.5) (layer "F.Cu") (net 1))
 (segment (start 201.855611 88.019611) (end 205.731389 88.019611) (width 2.5) (layer "F.Cu") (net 1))
 (segment (start 205.737857 107.954848) (end 205.735152 107.954848) (width 2.5) (layer "F.Cu") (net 1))
 (segment (start 201.854 88.018) (end 201.855611 88.019611) (width 2.5) (layer "F.Cu") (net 1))
 (segment (start 201.7595 109.22) (end 201.6565 109.117) (width 2.5) (layer "B.Cu") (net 1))
 (segment (start 204.47 109.22) (end 201.7595 109.22) (width 2.5) (layer "B.Cu") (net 1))
 (segment (start 205.74 107.95) (end 204.47 109.22) (width 2.5) (layer "B.Cu") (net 1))
 (segment (start 205.74 88.011) (end 205.74 107.95) (width 2.5) (layer "B.Cu") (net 1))
 (segment (start 201.854 88.018) (end 205.733 88.018) (width 2.5) (layer "B.Cu") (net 1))
 (segment (start 197.231 83.312) (end 197.231 90.805) (width 2.5) (layer "F.Cu") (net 2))
 (segment (start 186.436 90.678) (end 186.436 88.891) (width 2.5) (layer "F.Cu") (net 2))
 (segment (start 168.021 88.764) (end 169.935 90.678) (width 2.5) (layer "F.Cu") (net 2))
 (segment (start 201.854 83.018) (end 201.814 83.058) (width 2.5) (layer "F.Cu") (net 2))
 (segment (start 201.814 83.058) (end 197.485 83.058) (width 2.5) (layer "F.Cu") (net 2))
 (segment (start 197.231 119.846) (end 197.252 119.867) (width 2.5) (layer "F.Cu") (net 2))
 (segment (start 197.104 90.678) (end 197.231 90.805) (width 2.5) (layer "F.Cu") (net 2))
 (segment (start 169.935 90.678) (end 186.436 90.678) (width 2.5) (layer "F.Cu") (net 2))
 (segment (start 197.252 119.867) (end 201.6565 119.867) (width 2.5) (layer "F.Cu") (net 2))
 (segment (start 186.436 88.891) (end 186.309 88.764) (width 2.5) (layer "F.Cu") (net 2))
 (segment (start 197.485 83.058) (end 197.231 83.312) (width 2.5) (layer "F.Cu") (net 2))
 (segment (start 197.231 90.805) (end 197.231 119.846) (width 2.5) (layer "F.Cu") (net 2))
 (segment (start 186.436 90.678) (end 197.104 90.678) (width 2.5) (layer "F.Cu") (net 2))
 (segment (start 169.935 90.678) (end 186.309 90.678) (width 2.5) (layer "B.Cu") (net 2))
 (segment (start 197.231 83.312) (end 197.485 83.058) (width 2.5) (layer "B.Cu") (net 2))
 (segment (start 197.252 119.867) (end 197.231 119.846) (width 2.5) (layer "B.Cu") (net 2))
 (segment (start 197.231 119.846) (end 197.231 90.678) (width 2.5) (layer "B.Cu") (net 2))
 (segment (start 201.814 83.058) (end 201.854 83.018) (width 2.5) (layer "B.Cu") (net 2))
 (segment (start 201.6565 119.867) (end 197.252 119.867) (width 2.5) (layer "B.Cu") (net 2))
 (segment (start 197.231 90.678) (end 197.231 83.312) (width 2.5) (layer "B.Cu") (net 2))
 (segment (start 197.485 83.058) (end 201.814 83.058) (width 2.5) (layer "B.Cu") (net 2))
 (segment (start 186.309 88.764) (end 186.309 90.678) (width 2.5) (layer "B.Cu") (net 2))
 (segment (start 186.309 90.678) (end 197.231 90.678) (width 2.5) (layer "B.Cu") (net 2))
 (segment (start 168.021 88.764) (end 169.935 90.678) (width 2.5) (layer "B.Cu") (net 2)))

